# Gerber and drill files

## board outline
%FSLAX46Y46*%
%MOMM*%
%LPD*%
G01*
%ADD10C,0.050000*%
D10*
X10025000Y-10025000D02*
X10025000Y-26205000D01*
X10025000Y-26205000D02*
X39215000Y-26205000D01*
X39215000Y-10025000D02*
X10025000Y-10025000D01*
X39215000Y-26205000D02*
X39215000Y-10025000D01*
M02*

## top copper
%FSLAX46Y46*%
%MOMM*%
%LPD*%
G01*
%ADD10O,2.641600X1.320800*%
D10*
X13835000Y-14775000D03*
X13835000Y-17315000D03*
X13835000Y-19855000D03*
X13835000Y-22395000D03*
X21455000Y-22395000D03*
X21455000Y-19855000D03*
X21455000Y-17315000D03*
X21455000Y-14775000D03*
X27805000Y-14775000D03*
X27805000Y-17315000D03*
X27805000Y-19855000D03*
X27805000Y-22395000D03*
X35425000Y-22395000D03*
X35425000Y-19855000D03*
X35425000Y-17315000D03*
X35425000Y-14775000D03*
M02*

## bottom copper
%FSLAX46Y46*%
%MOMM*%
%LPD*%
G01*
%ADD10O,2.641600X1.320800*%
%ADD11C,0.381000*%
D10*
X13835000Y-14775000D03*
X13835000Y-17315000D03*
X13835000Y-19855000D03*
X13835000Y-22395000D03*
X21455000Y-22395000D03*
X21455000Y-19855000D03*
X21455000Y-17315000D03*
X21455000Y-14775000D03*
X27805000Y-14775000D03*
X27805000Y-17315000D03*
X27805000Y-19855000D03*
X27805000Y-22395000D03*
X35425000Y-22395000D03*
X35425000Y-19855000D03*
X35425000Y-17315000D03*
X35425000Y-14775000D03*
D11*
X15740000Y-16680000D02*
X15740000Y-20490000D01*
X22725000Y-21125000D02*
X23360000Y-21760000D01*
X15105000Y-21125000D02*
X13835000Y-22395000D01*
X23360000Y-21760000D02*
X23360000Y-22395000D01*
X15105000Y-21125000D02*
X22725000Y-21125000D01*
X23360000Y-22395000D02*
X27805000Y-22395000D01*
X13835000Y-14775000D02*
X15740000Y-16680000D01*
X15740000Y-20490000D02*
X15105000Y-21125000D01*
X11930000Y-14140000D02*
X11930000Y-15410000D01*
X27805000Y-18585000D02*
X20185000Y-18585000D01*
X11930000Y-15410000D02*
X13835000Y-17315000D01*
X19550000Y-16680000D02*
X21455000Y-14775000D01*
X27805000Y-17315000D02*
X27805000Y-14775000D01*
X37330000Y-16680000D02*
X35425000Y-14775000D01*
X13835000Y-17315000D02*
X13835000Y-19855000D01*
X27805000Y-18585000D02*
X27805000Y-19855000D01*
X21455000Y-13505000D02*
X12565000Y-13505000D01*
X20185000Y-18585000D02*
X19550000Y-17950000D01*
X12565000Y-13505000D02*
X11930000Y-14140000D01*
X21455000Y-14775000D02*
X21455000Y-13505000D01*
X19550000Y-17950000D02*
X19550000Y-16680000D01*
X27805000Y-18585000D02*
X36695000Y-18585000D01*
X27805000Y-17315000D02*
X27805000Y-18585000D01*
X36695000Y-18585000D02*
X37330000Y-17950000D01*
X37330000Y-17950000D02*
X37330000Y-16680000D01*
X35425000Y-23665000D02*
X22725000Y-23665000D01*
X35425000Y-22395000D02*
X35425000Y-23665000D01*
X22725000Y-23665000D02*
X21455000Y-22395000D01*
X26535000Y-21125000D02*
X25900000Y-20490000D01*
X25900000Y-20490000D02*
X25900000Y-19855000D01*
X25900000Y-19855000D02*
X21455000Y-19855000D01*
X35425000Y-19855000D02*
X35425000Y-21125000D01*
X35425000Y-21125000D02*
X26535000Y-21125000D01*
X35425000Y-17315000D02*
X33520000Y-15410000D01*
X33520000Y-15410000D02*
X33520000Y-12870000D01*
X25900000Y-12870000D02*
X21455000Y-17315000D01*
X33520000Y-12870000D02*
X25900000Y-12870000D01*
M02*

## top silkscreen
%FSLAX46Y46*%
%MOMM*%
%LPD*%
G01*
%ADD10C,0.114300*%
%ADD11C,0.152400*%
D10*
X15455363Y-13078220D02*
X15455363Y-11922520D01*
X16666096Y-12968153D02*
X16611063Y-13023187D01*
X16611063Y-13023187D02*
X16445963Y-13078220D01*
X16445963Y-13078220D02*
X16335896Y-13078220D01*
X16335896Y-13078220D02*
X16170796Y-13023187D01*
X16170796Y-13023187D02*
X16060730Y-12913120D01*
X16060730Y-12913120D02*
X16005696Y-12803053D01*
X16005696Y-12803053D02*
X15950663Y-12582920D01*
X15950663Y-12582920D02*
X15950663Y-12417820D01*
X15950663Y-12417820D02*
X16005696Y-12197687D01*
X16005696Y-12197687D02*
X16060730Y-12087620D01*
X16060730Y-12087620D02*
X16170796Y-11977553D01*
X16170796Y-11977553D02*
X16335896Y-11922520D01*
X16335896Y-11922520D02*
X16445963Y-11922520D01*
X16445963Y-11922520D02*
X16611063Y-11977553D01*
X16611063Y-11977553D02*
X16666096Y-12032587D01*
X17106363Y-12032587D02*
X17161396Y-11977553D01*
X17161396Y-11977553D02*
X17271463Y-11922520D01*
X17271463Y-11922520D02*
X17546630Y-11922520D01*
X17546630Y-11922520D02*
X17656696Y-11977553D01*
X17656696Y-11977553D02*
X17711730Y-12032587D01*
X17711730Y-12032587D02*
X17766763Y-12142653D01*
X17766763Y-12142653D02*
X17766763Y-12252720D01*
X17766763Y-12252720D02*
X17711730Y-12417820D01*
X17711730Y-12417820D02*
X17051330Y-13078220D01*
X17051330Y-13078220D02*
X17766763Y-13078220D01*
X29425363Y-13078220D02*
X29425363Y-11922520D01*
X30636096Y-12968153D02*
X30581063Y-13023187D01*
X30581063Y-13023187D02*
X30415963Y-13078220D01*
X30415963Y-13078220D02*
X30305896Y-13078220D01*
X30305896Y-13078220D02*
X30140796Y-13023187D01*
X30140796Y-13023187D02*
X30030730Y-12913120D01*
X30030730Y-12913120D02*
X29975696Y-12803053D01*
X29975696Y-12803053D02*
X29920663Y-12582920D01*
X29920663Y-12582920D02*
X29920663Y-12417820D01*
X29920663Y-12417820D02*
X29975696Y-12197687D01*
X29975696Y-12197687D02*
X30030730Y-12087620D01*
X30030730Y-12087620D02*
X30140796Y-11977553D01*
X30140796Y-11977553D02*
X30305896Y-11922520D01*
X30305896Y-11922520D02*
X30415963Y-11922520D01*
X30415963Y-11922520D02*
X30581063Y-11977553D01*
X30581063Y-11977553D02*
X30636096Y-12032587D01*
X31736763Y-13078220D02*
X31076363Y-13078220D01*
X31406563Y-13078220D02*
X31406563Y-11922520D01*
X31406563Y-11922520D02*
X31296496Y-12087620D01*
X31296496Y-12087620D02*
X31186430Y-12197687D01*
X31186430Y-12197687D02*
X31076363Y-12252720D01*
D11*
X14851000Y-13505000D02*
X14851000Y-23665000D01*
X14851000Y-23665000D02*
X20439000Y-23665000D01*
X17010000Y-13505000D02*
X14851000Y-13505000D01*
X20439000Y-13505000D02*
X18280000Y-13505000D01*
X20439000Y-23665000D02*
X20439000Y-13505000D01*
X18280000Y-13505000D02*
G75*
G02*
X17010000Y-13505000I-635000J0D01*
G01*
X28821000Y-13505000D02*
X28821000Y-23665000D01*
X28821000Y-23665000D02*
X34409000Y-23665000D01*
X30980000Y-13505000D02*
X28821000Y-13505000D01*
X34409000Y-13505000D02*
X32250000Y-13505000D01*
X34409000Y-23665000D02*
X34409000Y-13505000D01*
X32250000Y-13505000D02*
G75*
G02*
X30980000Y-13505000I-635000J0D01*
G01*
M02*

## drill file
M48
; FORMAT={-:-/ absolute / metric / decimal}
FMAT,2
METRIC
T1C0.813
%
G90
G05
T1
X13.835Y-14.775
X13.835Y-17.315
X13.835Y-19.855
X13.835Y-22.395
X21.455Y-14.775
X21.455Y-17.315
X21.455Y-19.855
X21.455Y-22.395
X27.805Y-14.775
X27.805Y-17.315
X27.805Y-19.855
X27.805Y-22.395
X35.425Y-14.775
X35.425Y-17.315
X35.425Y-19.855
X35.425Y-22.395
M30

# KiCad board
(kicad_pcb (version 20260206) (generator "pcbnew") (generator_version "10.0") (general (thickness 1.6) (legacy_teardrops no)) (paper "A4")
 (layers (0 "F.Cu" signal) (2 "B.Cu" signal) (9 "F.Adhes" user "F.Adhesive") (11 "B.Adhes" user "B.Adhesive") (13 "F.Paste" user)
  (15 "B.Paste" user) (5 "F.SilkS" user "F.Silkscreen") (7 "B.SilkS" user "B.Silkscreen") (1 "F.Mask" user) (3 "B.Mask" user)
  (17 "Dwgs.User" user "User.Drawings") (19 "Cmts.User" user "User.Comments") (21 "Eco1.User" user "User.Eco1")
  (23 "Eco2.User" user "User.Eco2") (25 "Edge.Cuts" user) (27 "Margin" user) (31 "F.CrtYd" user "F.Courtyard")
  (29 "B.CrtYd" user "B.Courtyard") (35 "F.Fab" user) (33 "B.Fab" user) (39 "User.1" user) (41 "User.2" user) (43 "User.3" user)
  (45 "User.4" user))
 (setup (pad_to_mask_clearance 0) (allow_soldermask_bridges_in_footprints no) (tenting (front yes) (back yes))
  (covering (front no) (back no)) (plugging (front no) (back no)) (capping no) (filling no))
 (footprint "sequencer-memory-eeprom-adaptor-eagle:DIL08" (layer "F.Cu") (at 17.645 18.585 -90)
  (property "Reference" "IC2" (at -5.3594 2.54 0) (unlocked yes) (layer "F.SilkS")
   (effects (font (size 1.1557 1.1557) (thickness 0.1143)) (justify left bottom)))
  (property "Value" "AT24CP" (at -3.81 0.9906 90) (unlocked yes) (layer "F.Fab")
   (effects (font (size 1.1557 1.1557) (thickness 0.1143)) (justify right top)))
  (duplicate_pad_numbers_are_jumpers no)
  (fp_line (start -5.08 2.794) (end 5.08 2.794) (stroke (width 0.1524) (type solid)) (layer "F.SilkS"))
  (fp_line (start 5.08 2.794) (end 5.08 -2.794) (stroke (width 0.1524) (type solid)) (layer "F.SilkS"))
  (fp_line (start -5.08 0.635) (end -5.08 2.794) (stroke (width 0.1524) (type solid)) (layer "F.SilkS"))
  (fp_line (start -5.08 -2.794) (end -5.08 -0.635) (stroke (width 0.1524) (type solid)) (layer "F.SilkS"))
  (fp_line (start 5.08 -2.794) (end -5.08 -2.794) (stroke (width 0.1524) (type solid)) (layer "F.SilkS"))
  (fp_arc (start -5.08 -0.635) (mid -4.445 0) (end -5.08 0.635) (stroke (width 0.1524) (type solid)) (layer "F.SilkS"))
  (pad "1" thru_hole oval (at -3.81 3.81) (size 2.6416 1.3208) (drill 0.8128) (layers "*.Cu" "*.Mask") (remove_unused_layers no) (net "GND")
   (solder_mask_margin 0.1016) (thermal_bridge_angle 0))
  (pad "2" thru_hole oval (at -1.27 3.81) (size 2.6416 1.3208) (drill 0.8128) (layers "*.Cu" "*.Mask") (remove_unused_layers no) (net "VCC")
   (solder_mask_margin 0.1016) (thermal_bridge_angle 0))
  (pad "3" thru_hole oval (at 1.27 3.81) (size 2.6416 1.3208) (drill 0.8128) (layers "*.Cu" "*.Mask") (remove_unused_layers no) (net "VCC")
   (solder_mask_margin 0.1016) (thermal_bridge_angle 0))
  (pad "4" thru_hole oval (at 3.81 3.81) (size 2.6416 1.3208) (drill 0.8128) (layers "*.Cu" "*.Mask") (remove_unused_layers no) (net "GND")
   (solder_mask_margin 0.1016) (thermal_bridge_angle 0))
  (pad "5" thru_hole oval (at 3.81 -3.81) (size 2.6416 1.3208) (drill 0.8128) (layers "*.Cu" "*.Mask") (remove_unused_layers no) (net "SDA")
   (solder_mask_margin 0.1016) (thermal_bridge_angle 0))
  (pad "6" thru_hole oval (at 1.27 -3.81) (size 2.6416 1.3208) (drill 0.8128) (layers "*.Cu" "*.Mask") (remove_unused_layers no) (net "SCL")
   (solder_mask_margin 0.1016) (thermal_bridge_angle 0))
  (pad "7" thru_hole oval (at -1.27 -3.81) (size 2.6416 1.3208) (drill 0.8128) (layers "*.Cu" "*.Mask") (remove_unused_layers no) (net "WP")
   (solder_mask_margin 0.1016) (thermal_bridge_angle 0))
  (pad "8" thru_hole oval (at -3.81 -3.81) (size 2.6416 1.3208) (drill 0.8128) (layers "*.Cu" "*.Mask") (remove_unused_layers no)
   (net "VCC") (solder_mask_margin 0.1016) (thermal_bridge_angle 0)))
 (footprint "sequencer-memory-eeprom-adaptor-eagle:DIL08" (layer "F.Cu") (at 31.615 18.585 -90)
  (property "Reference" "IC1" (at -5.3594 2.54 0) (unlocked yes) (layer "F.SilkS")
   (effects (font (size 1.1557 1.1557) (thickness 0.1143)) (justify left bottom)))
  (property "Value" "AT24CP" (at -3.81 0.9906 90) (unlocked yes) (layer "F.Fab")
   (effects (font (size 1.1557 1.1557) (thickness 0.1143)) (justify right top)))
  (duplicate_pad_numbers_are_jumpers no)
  (fp_line (start -5.08 2.794) (end 5.08 2.794) (stroke (width 0.1524) (type solid)) (layer "F.SilkS"))
  (fp_line (start 5.08 2.794) (end 5.08 -2.794) (stroke (width 0.1524) (type solid)) (layer "F.SilkS"))
  (fp_line (start -5.08 0.635) (end -5.08 2.794) (stroke (width 0.1524) (type solid)) (layer "F.SilkS"))
  (fp_line (start -5.08 -2.794) (end -5.08 -0.635) (stroke (width 0.1524) (type solid)) (layer "F.SilkS"))
  (fp_line (start 5.08 -2.794) (end -5.08 -2.794) (stroke (width 0.1524) (type solid)) (layer "F.SilkS"))
  (fp_arc (start -5.08 -0.635) (mid -4.445 0) (end -5.08 0.635) (stroke (width 0.1524) (type solid)) (layer "F.SilkS"))
  (pad "1" thru_hole oval (at -3.81 3.81) (size 2.6416 1.3208) (drill 0.8128) (layers "*.Cu" "*.Mask") (remove_unused_layers no) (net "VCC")
   (solder_mask_margin 0.1016) (thermal_bridge_angle 0))
  (pad "2" thru_hole oval (at -1.27 3.81) (size 2.6416 1.3208) (drill 0.8128) (layers "*.Cu" "*.Mask") (remove_unused_layers no) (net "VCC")
   (solder_mask_margin 0.1016) (thermal_bridge_angle 0))
  (pad "3" thru_hole oval (at 1.27 3.81) (size 2.6416 1.3208) (drill 0.8128) (layers "*.Cu" "*.Mask") (remove_unused_layers no) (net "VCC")
   (solder_mask_margin 0.1016) (thermal_bridge_angle 0))
  (pad "4" thru_hole oval (at 3.81 3.81) (size 2.6416 1.3208) (drill 0.8128) (layers "*.Cu" "*.Mask") (remove_unused_layers no) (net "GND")
   (solder_mask_margin 0.1016) (thermal_bridge_angle 0))
  (pad "5" thru_hole oval (at 3.81 -3.81) (size 2.6416 1.3208) (drill 0.8128) (layers "*.Cu" "*.Mask") (remove_unused_layers no) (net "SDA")
   (solder_mask_margin 0.1016) (thermal_bridge_angle 0))
  (pad "6" thru_hole oval (at 1.27 -3.81) (size 2.6416 1.3208) (drill 0.8128) (layers "*.Cu" "*.Mask") (remove_unused_layers no) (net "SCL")
   (solder_mask_margin 0.1016) (thermal_bridge_angle 0))
  (pad "7" thru_hole oval (at -1.27 -3.81) (size 2.6416 1.3208) (drill 0.8128) (layers "*.Cu" "*.Mask") (remove_unused_layers no) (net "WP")
   (solder_mask_margin 0.1016) (thermal_bridge_angle 0))
  (pad "8" thru_hole oval (at -3.81 -3.81) (size 2.6416 1.3208) (drill 0.8128) (layers "*.Cu" "*.Mask") (remove_unused_layers no)
   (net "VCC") (solder_mask_margin 0.1016) (thermal_bridge_angle 0)))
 (gr_line (start 10.025 10.025) (end 10.025 26.205) (stroke (width 0.05) (type solid)) (layer "Edge.Cuts"))
 (gr_line (start 10.025 26.205) (end 39.215 26.205) (stroke (width 0.05) (type solid)) (layer "Edge.Cuts"))
 (gr_line (start 39.215 10.025) (end 10.025 10.025) (stroke (width 0.05) (type solid)) (layer "Edge.Cuts"))
 (gr_line (start 39.215 26.205) (end 39.215 10.025) (stroke (width 0.05) (type solid)) (layer "Edge.Cuts"))
 (segment (start 15.74 16.68) (end 15.74 20.49) (width 0.381) (layer "B.Cu") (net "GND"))
 (segment (start 22.725 21.125) (end 23.36 21.76) (width 0.381) (layer "B.Cu") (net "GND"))
 (segment (start 15.105 21.125) (end 13.835 22.395) (width 0.381) (layer "B.Cu") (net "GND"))
 (segment (start 23.36 21.76) (end 23.36 22.395) (width 0.381) (layer "B.Cu") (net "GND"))
 (segment (start 15.105 21.125) (end 22.725 21.125) (width 0.381) (layer "B.Cu") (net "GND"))
 (segment (start 23.36 22.395) (end 27.805 22.395) (width 0.381) (layer "B.Cu") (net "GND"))
 (segment (start 13.835 14.775) (end 15.74 16.68) (width 0.381) (layer "B.Cu") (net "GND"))
 (segment (start 15.74 20.49) (end 15.105 21.125) (width 0.381) (layer "B.Cu") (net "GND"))
 (segment (start 11.93 14.14) (end 11.93 15.41) (width 0.381) (layer "B.Cu") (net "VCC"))
 (segment (start 27.805 18.585) (end 20.185 18.585) (width 0.381) (layer "B.Cu") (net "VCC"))
 (segment (start 11.93 15.41) (end 13.835 17.315) (width 0.381) (layer "B.Cu") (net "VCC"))
 (segment (start 19.55 16.68) (end 21.455 14.775) (width 0.381) (layer "B.Cu") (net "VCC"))
 (segment (start 27.805 17.315) (end 27.805 14.775) (width 0.381) (layer "B.Cu") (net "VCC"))
 (segment (start 37.33 16.68) (end 35.425 14.775) (width 0.381) (layer "B.Cu") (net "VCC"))
 (segment (start 13.835 17.315) (end 13.835 19.855) (width 0.381) (layer "B.Cu") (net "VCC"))
 (segment (start 27.805 18.585) (end 27.805 19.855) (width 0.381) (layer "B.Cu") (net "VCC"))
 (segment (start 21.455 13.505) (end 12.565 13.505) (width 0.381) (layer "B.Cu") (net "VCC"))
 (segment (start 20.185 18.585) (end 19.55 17.95) (width 0.381) (layer "B.Cu") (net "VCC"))
 (segment (start 12.565 13.505) (end 11.93 14.14) (width 0.381) (layer "B.Cu") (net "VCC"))
 (segment (start 21.455 14.775) (end 21.455 13.505) (width 0.381) (layer "B.Cu") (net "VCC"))
 (segment (start 19.55 17.95) (end 19.55 16.68) (width 0.381) (layer "B.Cu") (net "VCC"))
 (segment (start 27.805 18.585) (end 36.695 18.585) (width 0.381) (layer "B.Cu") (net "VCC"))
 (segment (start 27.805 17.315) (end 27.805 18.585) (width 0.381) (layer "B.Cu") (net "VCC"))
 (segment (start 36.695 18.585) (end 37.33 17.95) (width 0.381) (layer "B.Cu") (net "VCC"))
 (segment (start 37.33 17.95) (end 37.33 16.68) (width 0.381) (layer "B.Cu") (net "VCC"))
 (segment (start 35.425 23.665) (end 22.725 23.665) (width 0.381) (layer "B.Cu") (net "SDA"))
 (segment (start 35.425 22.395) (end 35.425 23.665) (width 0.381) (layer "B.Cu") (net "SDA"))
 (segment (start 22.725 23.665) (end 21.455 22.395) (width 0.381) (layer "B.Cu") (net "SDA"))
 (segment (start 26.535 21.125) (end 25.9 20.49) (width 0.381) (layer "B.Cu") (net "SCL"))
 (segment (start 25.9 20.49) (end 25.9 19.855) (width 0.381) (layer "B.Cu") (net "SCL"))
 (segment (start 25.9 19.855) (end 21.455 19.855) (width 0.381) (layer "B.Cu") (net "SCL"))
 (segment (start 35.425 19.855) (end 35.425 21.125) (width 0.381) (layer "B.Cu") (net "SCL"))
 (segment (start 35.425 21.125) (end 26.535 21.125) (width 0.381) (layer "B.Cu") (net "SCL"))
 (segment (start 35.425 17.315) (end 33.52 15.41) (width 0.381) (layer "B.Cu") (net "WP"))
 (segment (start 33.52 15.41) (end 33.52 12.87) (width 0.381) (layer "B.Cu") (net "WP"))
 (segment (start 25.9 12.87) (end 21.455 17.315) (width 0.381) (layer "B.Cu") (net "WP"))
 (segment (start 33.52 12.87) (end 25.9 12.87) (width 0.381) (layer "B.Cu") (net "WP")))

